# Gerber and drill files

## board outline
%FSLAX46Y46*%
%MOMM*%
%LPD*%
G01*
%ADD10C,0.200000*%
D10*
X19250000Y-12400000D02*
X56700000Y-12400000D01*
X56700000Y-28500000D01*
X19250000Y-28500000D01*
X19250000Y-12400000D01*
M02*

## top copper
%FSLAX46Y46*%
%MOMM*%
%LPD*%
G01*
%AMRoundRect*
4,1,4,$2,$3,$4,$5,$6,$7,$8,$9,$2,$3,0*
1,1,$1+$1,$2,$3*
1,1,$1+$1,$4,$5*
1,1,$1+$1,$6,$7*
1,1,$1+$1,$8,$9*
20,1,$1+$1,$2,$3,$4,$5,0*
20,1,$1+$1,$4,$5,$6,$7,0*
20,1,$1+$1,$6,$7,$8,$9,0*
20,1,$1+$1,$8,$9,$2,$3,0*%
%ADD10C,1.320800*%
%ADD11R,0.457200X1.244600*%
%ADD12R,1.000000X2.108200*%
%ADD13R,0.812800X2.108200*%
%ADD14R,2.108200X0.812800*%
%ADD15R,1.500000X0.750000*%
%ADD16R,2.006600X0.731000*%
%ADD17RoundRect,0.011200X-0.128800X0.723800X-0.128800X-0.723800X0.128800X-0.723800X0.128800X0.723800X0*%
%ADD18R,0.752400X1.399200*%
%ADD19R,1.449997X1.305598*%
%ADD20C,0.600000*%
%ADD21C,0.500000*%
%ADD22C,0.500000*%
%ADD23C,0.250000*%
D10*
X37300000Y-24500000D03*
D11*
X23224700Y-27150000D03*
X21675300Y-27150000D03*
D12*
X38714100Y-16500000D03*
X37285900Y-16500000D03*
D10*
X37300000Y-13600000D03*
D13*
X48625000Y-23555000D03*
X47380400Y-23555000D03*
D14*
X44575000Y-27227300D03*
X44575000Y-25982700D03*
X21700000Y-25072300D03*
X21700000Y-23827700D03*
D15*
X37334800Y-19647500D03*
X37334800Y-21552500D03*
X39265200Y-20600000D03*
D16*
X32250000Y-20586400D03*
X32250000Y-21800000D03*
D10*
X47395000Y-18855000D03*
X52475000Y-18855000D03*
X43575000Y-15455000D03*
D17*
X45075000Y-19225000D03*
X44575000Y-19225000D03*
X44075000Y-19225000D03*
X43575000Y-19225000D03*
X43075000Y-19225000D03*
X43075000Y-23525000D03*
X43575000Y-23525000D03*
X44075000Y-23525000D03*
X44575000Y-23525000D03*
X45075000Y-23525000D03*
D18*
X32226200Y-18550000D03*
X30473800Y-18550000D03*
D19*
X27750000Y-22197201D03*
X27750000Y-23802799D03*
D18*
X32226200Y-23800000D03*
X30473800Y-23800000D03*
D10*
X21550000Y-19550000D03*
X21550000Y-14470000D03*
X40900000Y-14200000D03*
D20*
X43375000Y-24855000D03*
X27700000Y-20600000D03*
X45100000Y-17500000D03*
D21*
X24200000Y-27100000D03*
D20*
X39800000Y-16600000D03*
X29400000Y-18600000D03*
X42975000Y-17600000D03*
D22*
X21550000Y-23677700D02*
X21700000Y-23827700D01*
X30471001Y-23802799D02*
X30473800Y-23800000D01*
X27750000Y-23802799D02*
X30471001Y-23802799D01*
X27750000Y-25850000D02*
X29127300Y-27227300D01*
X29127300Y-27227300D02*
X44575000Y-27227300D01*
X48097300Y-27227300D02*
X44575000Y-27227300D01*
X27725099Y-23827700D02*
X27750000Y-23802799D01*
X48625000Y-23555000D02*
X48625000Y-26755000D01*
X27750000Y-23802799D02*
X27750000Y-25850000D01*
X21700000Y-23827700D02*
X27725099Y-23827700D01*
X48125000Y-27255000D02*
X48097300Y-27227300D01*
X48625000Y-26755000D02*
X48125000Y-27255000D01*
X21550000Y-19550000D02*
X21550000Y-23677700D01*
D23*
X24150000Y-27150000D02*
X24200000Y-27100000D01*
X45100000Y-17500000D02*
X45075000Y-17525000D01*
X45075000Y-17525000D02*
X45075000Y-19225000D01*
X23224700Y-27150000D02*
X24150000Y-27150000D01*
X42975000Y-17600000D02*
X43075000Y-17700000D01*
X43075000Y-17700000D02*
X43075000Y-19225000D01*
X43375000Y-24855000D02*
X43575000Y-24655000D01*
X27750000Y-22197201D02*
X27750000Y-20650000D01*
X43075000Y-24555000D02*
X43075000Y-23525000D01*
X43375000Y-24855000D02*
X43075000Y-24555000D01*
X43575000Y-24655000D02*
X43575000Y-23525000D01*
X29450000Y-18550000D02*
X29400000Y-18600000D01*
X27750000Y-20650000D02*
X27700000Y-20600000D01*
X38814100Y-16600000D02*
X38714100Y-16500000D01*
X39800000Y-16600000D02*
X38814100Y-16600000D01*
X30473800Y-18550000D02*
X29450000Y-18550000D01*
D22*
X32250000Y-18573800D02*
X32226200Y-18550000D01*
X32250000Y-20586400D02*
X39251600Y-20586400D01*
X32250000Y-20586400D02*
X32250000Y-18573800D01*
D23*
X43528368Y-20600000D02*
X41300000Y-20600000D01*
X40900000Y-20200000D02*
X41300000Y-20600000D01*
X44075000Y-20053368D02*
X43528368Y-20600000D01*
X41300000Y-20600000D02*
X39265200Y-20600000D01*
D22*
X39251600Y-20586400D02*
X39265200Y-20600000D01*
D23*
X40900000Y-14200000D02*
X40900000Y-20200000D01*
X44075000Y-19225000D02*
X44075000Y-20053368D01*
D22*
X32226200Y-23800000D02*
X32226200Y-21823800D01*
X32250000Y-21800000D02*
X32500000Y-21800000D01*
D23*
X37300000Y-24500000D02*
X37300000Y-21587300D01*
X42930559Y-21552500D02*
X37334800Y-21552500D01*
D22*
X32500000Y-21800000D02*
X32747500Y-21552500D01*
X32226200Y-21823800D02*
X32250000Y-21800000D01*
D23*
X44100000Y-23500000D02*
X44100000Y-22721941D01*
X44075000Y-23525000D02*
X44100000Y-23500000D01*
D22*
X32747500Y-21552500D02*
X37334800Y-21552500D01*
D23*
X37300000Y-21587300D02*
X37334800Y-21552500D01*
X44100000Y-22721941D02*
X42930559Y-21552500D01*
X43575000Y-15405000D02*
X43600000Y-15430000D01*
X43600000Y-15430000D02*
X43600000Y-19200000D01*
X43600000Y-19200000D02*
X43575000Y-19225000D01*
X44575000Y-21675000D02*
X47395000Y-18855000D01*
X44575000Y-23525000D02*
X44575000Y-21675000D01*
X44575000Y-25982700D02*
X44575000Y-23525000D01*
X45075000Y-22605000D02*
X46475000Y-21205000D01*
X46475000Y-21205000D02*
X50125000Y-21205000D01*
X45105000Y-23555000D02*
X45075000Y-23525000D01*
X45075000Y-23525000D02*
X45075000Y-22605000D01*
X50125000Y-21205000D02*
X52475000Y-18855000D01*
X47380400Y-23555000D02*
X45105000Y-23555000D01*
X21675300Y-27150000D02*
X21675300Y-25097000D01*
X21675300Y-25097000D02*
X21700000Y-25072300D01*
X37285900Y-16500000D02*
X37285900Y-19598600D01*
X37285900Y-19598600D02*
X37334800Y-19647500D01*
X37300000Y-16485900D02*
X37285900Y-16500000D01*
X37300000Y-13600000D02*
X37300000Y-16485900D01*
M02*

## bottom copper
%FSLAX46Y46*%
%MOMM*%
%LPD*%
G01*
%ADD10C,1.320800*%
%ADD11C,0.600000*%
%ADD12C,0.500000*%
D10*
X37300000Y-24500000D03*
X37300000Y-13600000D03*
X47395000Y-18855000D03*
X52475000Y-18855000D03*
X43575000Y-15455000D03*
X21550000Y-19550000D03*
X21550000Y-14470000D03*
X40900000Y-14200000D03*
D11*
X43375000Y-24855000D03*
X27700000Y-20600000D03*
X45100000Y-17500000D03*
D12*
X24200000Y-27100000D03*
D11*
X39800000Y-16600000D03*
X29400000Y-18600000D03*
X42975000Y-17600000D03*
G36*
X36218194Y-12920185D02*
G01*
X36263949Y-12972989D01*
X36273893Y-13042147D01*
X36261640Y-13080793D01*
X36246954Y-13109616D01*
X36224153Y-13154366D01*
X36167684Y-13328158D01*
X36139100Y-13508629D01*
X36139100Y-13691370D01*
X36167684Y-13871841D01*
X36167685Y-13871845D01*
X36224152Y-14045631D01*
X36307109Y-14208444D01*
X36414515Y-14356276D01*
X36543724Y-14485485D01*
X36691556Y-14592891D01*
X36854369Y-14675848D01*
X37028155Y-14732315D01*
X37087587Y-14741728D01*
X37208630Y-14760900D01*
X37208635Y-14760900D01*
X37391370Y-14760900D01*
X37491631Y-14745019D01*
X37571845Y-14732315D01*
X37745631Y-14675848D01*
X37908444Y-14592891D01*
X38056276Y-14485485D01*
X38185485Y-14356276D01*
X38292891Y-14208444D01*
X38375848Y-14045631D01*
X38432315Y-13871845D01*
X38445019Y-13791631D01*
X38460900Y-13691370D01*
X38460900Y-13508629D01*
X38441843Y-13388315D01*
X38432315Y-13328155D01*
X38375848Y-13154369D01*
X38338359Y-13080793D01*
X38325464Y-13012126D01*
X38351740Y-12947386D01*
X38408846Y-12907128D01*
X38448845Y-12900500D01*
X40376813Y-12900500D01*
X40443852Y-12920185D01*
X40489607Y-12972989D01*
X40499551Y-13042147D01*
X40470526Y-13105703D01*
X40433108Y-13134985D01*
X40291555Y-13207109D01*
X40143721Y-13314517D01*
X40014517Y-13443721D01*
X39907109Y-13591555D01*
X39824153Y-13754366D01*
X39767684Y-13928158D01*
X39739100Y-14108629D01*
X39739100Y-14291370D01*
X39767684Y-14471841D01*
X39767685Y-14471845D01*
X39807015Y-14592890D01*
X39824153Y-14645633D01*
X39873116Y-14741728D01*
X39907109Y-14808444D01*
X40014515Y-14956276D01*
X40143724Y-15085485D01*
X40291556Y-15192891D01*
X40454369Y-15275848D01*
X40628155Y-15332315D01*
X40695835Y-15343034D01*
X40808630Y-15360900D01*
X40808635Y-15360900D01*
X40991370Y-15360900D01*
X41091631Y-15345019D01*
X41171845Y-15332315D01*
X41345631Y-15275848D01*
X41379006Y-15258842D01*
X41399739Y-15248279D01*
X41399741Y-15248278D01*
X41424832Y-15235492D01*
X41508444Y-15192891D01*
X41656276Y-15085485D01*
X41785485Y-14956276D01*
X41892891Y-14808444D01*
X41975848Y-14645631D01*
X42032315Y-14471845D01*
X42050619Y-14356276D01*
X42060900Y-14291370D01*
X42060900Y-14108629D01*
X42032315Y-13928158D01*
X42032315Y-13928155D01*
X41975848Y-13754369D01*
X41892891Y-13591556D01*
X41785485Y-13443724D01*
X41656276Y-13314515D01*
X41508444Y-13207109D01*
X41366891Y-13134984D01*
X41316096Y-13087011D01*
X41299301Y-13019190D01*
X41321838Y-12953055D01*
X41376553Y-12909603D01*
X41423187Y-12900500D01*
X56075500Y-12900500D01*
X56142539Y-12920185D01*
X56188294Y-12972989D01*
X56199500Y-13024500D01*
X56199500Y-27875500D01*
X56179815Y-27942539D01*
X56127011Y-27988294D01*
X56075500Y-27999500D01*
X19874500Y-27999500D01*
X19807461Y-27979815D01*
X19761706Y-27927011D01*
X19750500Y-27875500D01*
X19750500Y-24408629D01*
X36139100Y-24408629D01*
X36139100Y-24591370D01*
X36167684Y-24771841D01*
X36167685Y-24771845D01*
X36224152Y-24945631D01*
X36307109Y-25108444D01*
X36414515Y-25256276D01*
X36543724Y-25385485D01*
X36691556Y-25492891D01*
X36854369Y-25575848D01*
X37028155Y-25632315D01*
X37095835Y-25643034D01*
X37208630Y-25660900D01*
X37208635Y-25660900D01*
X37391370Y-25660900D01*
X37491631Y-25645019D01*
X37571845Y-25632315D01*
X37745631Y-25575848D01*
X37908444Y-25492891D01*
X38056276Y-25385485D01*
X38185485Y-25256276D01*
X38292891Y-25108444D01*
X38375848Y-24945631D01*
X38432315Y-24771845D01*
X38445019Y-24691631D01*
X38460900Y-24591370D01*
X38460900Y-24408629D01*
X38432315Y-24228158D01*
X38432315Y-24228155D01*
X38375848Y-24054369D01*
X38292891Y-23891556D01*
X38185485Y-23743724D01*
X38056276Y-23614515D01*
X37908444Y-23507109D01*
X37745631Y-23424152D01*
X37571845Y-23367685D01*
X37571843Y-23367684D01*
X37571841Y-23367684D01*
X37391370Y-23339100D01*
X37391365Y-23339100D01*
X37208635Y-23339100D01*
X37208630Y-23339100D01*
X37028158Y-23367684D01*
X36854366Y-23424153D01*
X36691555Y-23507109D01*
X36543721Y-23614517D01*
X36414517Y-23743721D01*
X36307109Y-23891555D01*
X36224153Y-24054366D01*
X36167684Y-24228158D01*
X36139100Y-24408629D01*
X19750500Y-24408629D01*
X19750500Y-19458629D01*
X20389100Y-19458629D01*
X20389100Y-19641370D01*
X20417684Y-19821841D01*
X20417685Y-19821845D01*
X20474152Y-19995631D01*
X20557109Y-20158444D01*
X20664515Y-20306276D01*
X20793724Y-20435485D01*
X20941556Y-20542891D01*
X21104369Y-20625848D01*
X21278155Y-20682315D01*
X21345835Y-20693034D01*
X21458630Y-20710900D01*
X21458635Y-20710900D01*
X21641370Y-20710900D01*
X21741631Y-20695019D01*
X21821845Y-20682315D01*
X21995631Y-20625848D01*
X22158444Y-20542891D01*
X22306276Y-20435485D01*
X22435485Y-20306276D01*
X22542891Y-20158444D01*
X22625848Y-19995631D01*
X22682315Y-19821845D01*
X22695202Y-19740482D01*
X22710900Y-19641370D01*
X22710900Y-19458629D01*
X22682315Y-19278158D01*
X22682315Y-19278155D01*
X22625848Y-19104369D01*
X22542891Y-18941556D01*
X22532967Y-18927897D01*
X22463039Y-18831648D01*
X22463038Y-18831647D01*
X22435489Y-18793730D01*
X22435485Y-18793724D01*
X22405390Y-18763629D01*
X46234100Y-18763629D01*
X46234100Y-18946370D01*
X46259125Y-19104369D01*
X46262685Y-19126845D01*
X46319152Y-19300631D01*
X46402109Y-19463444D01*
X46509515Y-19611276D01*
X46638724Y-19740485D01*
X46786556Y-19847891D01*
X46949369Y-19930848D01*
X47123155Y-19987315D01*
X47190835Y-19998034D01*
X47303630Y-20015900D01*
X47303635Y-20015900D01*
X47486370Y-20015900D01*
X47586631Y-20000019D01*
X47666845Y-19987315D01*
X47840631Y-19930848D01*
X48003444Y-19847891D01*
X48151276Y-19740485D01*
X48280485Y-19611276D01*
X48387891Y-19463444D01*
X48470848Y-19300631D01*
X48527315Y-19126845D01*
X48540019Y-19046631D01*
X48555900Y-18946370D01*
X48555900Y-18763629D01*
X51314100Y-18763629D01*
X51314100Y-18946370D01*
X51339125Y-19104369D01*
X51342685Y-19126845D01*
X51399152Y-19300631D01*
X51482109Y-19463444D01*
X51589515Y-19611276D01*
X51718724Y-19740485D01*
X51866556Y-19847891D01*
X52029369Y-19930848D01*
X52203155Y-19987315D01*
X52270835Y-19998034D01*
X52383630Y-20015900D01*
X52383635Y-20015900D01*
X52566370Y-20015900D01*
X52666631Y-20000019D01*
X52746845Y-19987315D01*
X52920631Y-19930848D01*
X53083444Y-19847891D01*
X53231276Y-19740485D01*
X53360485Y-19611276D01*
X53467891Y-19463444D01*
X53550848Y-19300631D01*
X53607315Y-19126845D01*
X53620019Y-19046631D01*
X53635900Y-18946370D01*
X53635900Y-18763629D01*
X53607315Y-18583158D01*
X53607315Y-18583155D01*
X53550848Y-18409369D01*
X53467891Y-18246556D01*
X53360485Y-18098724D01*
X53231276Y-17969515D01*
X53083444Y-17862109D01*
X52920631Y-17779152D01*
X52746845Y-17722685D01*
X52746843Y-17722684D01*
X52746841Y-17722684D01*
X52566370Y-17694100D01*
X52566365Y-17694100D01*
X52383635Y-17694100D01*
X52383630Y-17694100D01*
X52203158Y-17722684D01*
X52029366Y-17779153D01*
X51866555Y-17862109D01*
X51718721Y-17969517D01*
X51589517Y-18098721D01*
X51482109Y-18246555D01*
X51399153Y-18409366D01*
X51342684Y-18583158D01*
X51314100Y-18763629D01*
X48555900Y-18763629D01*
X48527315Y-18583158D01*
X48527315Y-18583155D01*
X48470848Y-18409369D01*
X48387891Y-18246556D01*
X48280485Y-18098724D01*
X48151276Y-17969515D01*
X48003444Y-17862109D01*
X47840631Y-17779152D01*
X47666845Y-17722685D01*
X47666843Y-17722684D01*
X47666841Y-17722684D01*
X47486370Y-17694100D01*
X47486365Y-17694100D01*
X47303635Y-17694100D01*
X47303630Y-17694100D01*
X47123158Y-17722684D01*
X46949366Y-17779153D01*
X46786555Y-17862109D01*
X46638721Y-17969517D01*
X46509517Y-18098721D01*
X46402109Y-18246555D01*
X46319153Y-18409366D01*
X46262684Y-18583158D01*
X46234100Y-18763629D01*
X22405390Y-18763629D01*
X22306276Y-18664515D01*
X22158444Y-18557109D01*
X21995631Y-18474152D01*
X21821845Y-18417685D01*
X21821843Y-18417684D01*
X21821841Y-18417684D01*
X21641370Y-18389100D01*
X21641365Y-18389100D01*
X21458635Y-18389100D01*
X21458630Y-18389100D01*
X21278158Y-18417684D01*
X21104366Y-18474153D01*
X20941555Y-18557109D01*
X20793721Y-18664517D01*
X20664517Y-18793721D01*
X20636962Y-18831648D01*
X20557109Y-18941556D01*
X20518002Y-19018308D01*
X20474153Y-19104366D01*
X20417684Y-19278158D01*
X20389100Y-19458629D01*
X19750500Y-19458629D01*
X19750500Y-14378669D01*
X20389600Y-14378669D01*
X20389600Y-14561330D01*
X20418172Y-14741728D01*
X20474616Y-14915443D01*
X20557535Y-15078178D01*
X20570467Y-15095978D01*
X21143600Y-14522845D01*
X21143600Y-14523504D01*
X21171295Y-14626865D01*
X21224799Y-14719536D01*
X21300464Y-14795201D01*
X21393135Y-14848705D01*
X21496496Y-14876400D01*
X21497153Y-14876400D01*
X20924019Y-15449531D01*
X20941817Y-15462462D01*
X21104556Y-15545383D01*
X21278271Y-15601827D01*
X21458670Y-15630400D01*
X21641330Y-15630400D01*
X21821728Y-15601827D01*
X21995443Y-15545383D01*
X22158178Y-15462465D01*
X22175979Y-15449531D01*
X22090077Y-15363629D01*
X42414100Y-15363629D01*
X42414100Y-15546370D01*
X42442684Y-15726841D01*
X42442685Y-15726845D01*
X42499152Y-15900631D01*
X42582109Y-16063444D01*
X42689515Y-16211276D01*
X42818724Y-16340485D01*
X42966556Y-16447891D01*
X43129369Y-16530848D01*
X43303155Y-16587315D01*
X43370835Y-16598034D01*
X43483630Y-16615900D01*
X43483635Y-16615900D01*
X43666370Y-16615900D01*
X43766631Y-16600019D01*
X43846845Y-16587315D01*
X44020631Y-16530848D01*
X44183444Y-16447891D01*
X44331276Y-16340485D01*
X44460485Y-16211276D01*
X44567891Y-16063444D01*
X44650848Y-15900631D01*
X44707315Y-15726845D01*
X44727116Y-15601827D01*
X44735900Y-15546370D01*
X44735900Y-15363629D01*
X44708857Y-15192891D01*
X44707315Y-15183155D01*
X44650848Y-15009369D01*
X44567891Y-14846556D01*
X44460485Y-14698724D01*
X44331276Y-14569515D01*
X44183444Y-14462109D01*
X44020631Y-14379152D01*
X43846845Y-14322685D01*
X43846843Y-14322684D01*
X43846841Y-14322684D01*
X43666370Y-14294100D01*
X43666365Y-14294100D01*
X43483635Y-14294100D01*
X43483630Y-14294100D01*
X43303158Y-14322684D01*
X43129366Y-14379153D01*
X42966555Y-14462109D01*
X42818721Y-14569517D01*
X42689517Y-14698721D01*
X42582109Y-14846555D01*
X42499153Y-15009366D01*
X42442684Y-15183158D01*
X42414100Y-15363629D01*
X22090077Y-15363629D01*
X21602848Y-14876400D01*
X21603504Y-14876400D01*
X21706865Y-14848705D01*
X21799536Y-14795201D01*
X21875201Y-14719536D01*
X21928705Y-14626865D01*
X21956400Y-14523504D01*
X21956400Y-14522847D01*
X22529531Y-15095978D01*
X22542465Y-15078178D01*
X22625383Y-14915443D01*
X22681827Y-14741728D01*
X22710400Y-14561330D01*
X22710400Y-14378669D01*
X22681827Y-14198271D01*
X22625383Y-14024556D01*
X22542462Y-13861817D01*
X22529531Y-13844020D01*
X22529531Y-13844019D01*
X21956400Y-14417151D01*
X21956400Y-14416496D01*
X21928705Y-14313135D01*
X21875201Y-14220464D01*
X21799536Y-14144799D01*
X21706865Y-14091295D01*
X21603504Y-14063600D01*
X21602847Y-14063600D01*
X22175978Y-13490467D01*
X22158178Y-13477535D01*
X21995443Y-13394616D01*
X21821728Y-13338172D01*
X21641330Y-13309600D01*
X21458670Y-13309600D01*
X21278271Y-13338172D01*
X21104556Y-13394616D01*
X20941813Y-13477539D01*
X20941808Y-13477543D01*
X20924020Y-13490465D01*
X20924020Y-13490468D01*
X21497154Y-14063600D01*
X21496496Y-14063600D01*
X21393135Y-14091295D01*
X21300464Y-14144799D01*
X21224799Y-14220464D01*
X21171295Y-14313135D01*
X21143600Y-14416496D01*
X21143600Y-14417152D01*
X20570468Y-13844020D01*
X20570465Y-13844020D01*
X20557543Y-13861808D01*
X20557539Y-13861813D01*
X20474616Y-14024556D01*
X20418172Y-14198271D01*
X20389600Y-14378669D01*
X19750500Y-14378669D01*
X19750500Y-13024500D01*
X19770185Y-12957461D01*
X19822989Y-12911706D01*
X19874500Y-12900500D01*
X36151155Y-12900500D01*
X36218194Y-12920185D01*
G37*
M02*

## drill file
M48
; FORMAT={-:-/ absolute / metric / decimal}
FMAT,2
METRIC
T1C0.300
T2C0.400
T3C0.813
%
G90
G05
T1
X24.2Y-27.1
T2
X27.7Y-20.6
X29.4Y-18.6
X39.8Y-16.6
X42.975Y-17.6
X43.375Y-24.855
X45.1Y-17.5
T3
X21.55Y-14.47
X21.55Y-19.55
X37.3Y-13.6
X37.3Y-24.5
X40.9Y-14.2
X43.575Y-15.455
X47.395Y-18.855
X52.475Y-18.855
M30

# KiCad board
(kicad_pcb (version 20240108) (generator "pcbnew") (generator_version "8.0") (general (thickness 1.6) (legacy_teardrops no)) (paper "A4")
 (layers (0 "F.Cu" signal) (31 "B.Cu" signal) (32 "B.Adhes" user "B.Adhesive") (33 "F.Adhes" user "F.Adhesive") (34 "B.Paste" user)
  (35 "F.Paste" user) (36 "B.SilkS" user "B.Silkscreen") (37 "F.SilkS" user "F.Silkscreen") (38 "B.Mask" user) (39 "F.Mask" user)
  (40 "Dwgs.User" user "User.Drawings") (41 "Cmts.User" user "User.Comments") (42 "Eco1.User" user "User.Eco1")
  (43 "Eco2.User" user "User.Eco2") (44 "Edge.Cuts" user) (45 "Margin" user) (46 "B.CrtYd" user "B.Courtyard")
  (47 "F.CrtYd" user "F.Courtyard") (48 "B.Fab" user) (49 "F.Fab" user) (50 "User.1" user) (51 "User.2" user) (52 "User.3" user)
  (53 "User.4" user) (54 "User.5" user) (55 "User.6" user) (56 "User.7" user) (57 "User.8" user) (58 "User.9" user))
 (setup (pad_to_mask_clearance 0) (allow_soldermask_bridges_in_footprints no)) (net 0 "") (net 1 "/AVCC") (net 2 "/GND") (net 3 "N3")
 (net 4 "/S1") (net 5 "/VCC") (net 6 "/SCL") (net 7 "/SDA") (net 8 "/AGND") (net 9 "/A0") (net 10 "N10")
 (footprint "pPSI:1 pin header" (layer "F.Cu") (at 37.3 24.5)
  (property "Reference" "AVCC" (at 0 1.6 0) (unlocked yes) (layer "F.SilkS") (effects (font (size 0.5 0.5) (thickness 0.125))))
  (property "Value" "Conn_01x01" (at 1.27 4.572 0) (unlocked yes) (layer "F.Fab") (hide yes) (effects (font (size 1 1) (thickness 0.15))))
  (pad "1" thru_hole circle (at 0 0) (size 1.3208 1.3208) (drill 0.8128) (layers "*.Cu" "*.Mask") (remove_unused_layers no) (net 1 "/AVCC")))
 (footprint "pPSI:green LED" (layer "F.Cu") (at 22.45 27.15 180)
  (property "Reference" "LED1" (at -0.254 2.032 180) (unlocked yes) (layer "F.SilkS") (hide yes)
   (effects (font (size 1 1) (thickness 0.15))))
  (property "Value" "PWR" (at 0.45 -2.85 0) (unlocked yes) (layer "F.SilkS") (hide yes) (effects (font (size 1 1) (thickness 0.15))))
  (pad "1" smd rect (at -0.7747 0 180) (size 0.4572 1.2446) (layers "F.Cu" "F.Paste" "F.Mask") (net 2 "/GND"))
  (pad "2" smd rect (at 0.7747 0 180) (size 0.4572 1.2446) (layers "F.Cu" "F.Paste" "F.Mask") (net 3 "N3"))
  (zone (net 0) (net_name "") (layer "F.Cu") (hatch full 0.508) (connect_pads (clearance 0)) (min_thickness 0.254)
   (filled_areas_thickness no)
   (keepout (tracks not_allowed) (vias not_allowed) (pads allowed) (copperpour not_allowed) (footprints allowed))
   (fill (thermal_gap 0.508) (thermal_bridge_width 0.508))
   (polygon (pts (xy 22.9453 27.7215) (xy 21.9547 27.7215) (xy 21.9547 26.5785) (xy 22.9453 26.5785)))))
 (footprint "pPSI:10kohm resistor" (layer "F.Cu") (at 38 16.5 180)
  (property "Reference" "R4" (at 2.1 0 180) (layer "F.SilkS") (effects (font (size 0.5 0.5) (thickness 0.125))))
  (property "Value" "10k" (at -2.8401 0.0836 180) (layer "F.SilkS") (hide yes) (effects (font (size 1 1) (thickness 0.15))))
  (pad "1" smd rect (at -0.7141 0 180) (size 1 2.1082) (layers "F.Cu" "F.Paste" "F.Mask") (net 2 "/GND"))
  (pad "2" smd rect (at 0.7141 0 180) (size 1 2.1082) (layers "F.Cu" "F.Paste" "F.Mask") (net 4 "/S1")))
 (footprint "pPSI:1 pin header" (layer "F.Cu") (at 37.3 13.6 180)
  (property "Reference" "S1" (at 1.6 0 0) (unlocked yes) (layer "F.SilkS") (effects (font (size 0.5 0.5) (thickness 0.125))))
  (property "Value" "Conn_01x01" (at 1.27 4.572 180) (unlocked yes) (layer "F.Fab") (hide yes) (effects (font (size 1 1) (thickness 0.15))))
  (pad "1" thru_hole circle (at 0 0 180) (size 1.3208 1.3208) (drill 0.8128) (layers "*.Cu" "*.Mask") (remove_unused_layers no)
   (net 4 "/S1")))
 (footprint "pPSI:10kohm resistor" (layer "F.Cu") (at 48.0027 23.555 180)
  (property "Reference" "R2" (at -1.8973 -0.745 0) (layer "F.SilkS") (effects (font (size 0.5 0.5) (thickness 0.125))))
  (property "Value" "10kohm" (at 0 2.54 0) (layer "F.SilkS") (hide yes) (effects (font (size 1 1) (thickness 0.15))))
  (pad "1" smd rect (at -0.6223 0 180) (size 0.8128 2.1082) (layers "F.Cu" "F.Paste" "F.Mask") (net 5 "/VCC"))
  (pad "2" smd rect (at 0.6223 0 180) (size 0.8128 2.1082) (layers "F.Cu" "F.Paste" "F.Mask") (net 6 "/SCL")))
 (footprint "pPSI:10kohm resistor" (layer "F.Cu") (at 44.575 26.605 90)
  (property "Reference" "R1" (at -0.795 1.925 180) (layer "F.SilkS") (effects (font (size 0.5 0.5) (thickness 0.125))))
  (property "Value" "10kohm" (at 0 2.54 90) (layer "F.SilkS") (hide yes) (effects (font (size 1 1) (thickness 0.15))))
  (pad "1" smd rect (at -0.6223 0 90) (size 0.8128 2.1082) (layers "F.Cu" "F.Paste" "F.Mask") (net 5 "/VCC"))
  (pad "2" smd rect (at 0.6223 0 90) (size 0.8128 2.1082) (layers "F.Cu" "F.Paste" "F.Mask") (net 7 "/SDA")))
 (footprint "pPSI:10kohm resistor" (layer "F.Cu") (at 21.7 24.45 90)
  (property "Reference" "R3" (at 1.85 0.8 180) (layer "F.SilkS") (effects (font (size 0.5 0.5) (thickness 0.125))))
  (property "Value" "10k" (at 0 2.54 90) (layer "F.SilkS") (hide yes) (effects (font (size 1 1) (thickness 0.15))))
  (pad "1" smd rect (at -0.6223 0 90) (size 0.8128 2.1082) (layers "F.Cu" "F.Paste" "F.Mask") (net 3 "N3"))
  (pad "2" smd rect (at 0.6223 0 90) (size 0.8128 2.1082) (layers "F.Cu" "F.Paste" "F.Mask") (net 5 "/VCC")))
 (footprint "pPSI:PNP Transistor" (layer "F.Cu") (at 38.3 20.6 -90)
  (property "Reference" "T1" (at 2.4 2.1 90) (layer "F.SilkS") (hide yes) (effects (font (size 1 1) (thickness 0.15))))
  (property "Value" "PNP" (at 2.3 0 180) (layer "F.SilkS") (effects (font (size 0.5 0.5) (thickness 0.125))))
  (pad "1" smd rect (at -0.9525 0.9652 270) (size 0.75 1.5) (layers "F.Cu" "F.Paste" "F.Mask") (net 4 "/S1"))
  (pad "2" smd rect (at 0.9525 0.9652 270) (size 0.75 1.5) (layers "F.Cu" "F.Paste" "F.Mask") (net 1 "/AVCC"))
  (pad "3" smd rect (at 0 -0.9652 270) (size 0.75 1.5) (layers "F.Cu" "F.Paste" "F.Mask") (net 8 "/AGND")))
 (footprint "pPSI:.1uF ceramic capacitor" (layer "F.Cu") (at 32.25 21.1932 -90)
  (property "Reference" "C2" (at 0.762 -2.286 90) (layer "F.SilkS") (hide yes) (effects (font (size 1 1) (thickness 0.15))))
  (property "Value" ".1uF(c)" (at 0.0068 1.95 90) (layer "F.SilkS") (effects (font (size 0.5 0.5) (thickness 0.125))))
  (pad "1" smd rect (at -0.6068 0 270) (size 0.731 2.0066) (layers "F.Cu" "F.Paste" "F.Mask") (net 8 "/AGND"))
  (pad "2" smd rect (at 0.6068 0 270) (size 0.731 2.0066) (layers "F.Cu" "F.Paste" "F.Mask") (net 1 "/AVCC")))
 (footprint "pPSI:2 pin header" (layer "F.Cu") (at 47.395 18.855)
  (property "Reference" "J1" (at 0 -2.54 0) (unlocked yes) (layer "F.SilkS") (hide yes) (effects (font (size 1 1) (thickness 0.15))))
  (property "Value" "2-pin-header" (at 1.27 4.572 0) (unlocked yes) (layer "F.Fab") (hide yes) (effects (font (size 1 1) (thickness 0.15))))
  (pad "1" thru_hole circle (at 0 0) (size 1.3208 1.3208) (drill 0.8128) (layers "*.Cu" "*.Mask") (remove_unused_layers no) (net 7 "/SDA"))
  (pad "2" thru_hole circle (at 5.08 0) (size 1.3208 1.3208) (drill 0.8128) (layers "*.Cu" "*.Mask") (remove_unused_layers no)
   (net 6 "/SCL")))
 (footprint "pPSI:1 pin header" (layer "F.Cu") (at 43.575 15.455)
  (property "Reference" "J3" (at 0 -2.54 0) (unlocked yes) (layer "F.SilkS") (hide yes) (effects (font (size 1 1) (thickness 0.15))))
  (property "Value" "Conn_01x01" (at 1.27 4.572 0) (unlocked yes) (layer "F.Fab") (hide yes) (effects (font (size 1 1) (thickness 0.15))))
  (pad "1" thru_hole circle (at 0 0) (size 1.3208 1.3208) (drill 0.8128) (layers "*.Cu" "*.Mask") (remove_unused_layers no) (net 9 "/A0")))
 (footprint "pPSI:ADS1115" (layer "F.Cu") (at 44.075 21.375 -90)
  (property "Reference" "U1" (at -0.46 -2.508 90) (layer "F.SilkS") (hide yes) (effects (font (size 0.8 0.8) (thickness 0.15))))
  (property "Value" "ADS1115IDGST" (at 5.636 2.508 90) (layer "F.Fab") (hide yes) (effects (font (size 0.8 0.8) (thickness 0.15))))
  (pad "1" smd roundrect (at -2.15 -1 270) (size 1.47 0.28) (layers "F.Cu" "F.Paste" "F.Mask") (roundrect_rratio 0.04) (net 2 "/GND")
   (solder_mask_margin 0.102))
  (pad "2" smd roundrect (at -2.15 -0.5 270) (size 1.47 0.28) (layers "F.Cu" "F.Paste" "F.Mask") (roundrect_rratio 0.04) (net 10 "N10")
   (solder_mask_margin 0.102))
  (pad "3" smd roundrect (at -2.15 0 270) (size 1.47 0.28) (layers "F.Cu" "F.Paste" "F.Mask") (roundrect_rratio 0.04) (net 8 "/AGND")
   (solder_mask_margin 0.102))
  (pad "4" smd roundrect (at -2.15 0.5 270) (size 1.47 0.28) (layers "F.Cu" "F.Paste" "F.Mask") (roundrect_rratio 0.04) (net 9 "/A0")
   (solder_mask_margin 0.102))
  (pad "5" smd roundrect (at -2.15 1 270) (size 1.47 0.28) (layers "F.Cu" "F.Paste" "F.Mask") (roundrect_rratio 0.04) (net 2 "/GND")
   (solder_mask_margin 0.102))
  (pad "6" smd roundrect (at 2.15 1 270) (size 1.47 0.28) (layers "F.Cu" "F.Paste" "F.Mask") (roundrect_rratio 0.04) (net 2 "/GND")
   (solder_mask_margin 0.102))
  (pad "7" smd roundrect (at 2.15 0.5 270) (size 1.47 0.28) (layers "F.Cu" "F.Paste" "F.Mask") (roundrect_rratio 0.04) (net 2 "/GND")
   (solder_mask_margin 0.102))
  (pad "8" smd roundrect (at 2.15 0 270) (size 1.47 0.28) (layers "F.Cu" "F.Paste" "F.Mask") (roundrect_rratio 0.04) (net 1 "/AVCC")
   (solder_mask_margin 0.102))
  (pad "9" smd roundrect (at 2.15 -0.5 270) (size 1.47 0.28) (layers "F.Cu" "F.Paste" "F.Mask") (roundrect_rratio 0.04) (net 7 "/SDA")
   (solder_mask_margin 0.102))
  (pad "10" smd roundrect (at 2.15 -1 270) (size 1.47 0.28) (layers "F.Cu" "F.Paste" "F.Mask") (roundrect_rratio 0.04) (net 6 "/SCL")
   (solder_mask_margin 0.102)))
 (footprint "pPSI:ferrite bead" (layer "F.Cu") (at 31.35 18.55 180)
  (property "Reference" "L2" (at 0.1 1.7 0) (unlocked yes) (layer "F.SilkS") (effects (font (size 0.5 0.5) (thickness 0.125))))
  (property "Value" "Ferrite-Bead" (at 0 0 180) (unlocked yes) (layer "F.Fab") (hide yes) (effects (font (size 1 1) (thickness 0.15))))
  (pad "1" smd rect (at -0.8762 0 180) (size 0.7524 1.3992) (layers "F.Cu" "F.Paste" "F.Mask") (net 8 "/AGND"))
  (pad "2" smd rect (at 0.8762 0 180) (size 0.7524 1.3992) (layers "F.Cu" "F.Paste" "F.Mask") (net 2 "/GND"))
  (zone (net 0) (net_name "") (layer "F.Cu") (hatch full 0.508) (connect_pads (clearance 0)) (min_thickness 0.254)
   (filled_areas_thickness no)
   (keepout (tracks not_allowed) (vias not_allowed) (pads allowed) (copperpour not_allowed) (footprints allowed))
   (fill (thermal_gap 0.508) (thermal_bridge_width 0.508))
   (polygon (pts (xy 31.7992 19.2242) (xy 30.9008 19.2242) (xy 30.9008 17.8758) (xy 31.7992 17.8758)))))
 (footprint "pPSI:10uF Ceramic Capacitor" (layer "F.Cu") (at 27.75 23 -90)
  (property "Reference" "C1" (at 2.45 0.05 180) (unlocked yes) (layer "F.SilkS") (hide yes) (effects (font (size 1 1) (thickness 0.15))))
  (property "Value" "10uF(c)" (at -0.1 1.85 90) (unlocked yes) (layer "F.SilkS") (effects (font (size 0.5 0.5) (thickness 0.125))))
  (pad "1" smd rect (at -0.802799 0 270) (size 1.305598 1.449997) (layers "F.Cu" "F.Paste" "F.Mask") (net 2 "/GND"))
  (pad "2" smd rect (at 0.802799 0 270) (size 1.305598 1.449997) (layers "F.Cu" "F.Paste" "F.Mask") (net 5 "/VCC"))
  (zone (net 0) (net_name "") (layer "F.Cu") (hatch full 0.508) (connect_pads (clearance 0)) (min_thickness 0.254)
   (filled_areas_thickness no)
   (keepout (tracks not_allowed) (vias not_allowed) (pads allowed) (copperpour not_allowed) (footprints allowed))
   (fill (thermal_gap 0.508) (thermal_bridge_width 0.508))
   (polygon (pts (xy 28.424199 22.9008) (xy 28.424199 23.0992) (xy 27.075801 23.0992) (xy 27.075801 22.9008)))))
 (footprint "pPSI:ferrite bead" (layer "F.Cu") (at 31.35 23.8 180)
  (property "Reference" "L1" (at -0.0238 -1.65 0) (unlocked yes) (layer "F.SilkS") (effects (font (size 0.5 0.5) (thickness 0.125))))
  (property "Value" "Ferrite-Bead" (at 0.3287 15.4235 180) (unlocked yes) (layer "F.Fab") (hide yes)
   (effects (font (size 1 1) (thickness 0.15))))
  (pad "1" smd rect (at -0.8762 0 180) (size 0.7524 1.3992) (layers "F.Cu" "F.Paste" "F.Mask") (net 1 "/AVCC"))
  (pad "2" smd rect (at 0.8762 0 180) (size 0.7524 1.3992) (layers "F.Cu" "F.Paste" "F.Mask") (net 5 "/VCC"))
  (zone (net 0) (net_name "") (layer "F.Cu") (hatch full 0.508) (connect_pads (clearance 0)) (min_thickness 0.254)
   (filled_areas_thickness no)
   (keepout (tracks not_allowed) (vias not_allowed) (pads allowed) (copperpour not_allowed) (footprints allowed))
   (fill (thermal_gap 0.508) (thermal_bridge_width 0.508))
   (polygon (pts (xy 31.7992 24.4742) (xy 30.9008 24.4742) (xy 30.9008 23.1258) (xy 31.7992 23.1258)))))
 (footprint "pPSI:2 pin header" (layer "F.Cu") (at 21.55 19.55 90)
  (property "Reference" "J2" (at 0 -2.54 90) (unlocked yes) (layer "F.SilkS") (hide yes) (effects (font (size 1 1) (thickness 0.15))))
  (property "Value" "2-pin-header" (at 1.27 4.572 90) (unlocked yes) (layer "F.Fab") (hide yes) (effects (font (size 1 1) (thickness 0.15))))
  (pad "1" thru_hole circle (at 0 0 90) (size 1.3208 1.3208) (drill 0.8128) (layers "*.Cu" "*.Mask") (remove_unused_layers no)
   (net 5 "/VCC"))
  (pad "2" thru_hole circle (at 5.08 0 90) (size 1.3208 1.3208) (drill 0.8128) (layers "*.Cu" "*.Mask") (remove_unused_layers no)
   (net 2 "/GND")))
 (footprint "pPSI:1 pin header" (layer "F.Cu") (at 40.9 14.2 180)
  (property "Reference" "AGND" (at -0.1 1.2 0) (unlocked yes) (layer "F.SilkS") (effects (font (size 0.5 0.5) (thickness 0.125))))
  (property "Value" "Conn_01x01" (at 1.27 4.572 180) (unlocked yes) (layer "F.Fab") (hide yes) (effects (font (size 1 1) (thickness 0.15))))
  (pad "1" thru_hole circle (at 0 0 180) (size 1.3208 1.3208) (drill 0.8128) (layers "*.Cu" "*.Mask") (remove_unused_layers no)
   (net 8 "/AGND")))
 (gr_rect (start 19.25 12.4) (end 56.7 28.5) (stroke (width 0.2) (type solid)) (fill none) (layer "Edge.Cuts"))
 (segment (start 21.55 23.6777) (end 21.7 23.8277) (width 0.5) (layer "F.Cu") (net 5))
 (segment (start 30.471001 23.802799) (end 30.4738 23.8) (width 0.5) (layer "F.Cu") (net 5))
 (segment (start 27.75 23.802799) (end 30.471001 23.802799) (width 0.5) (layer "F.Cu") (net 5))
 (segment (start 27.75 25.85) (end 29.1273 27.2273) (width 0.5) (layer "F.Cu") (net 5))
 (segment (start 29.1273 27.2273) (end 44.575 27.2273) (width 0.5) (layer "F.Cu") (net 5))
 (segment (start 48.0973 27.2273) (end 44.575 27.2273) (width 0.5) (layer "F.Cu") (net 5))
 (segment (start 27.725099 23.8277) (end 27.75 23.802799) (width 0.5) (layer "F.Cu") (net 5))
 (segment (start 48.625 23.555) (end 48.625 26.755) (width 0.5) (layer "F.Cu") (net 5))
 (segment (start 27.75 23.802799) (end 27.75 25.85) (width 0.5) (layer "F.Cu") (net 5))
 (segment (start 21.7 23.8277) (end 27.725099 23.8277) (width 0.5) (layer "F.Cu") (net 5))
 (segment (start 48.125 27.255) (end 48.0973 27.2273) (width 0.5) (layer "F.Cu") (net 5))
 (segment (start 48.625 26.755) (end 48.125 27.255) (width 0.5) (layer "F.Cu") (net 5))
 (segment (start 21.55 19.55) (end 21.55 23.6777) (width 0.5) (layer "F.Cu") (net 5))
 (segment (start 24.15 27.15) (end 24.2 27.1) (width 0.25) (layer "F.Cu") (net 2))
 (segment (start 45.1 17.5) (end 45.075 17.525) (width 0.25) (layer "F.Cu") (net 2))
 (segment (start 45.075 17.525) (end 45.075 19.225) (width 0.25) (layer "F.Cu") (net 2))
 (segment (start 23.2247 27.15) (end 24.15 27.15) (width 0.25) (layer "F.Cu") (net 2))
 (segment (start 42.975 17.6) (end 43.075 17.7) (width 0.25) (layer "F.Cu") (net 2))
 (segment (start 43.075 17.7) (end 43.075 19.225) (width 0.25) (layer "F.Cu") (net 2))
 (segment (start 43.375 24.855) (end 43.575 24.655) (width 0.25) (layer "F.Cu") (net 2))
 (segment (start 27.75 22.197201) (end 27.75 20.65) (width 0.25) (layer "F.Cu") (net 2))
 (segment (start 43.075 24.555) (end 43.075 23.525) (width 0.25) (layer "F.Cu") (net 2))
 (segment (start 43.375 24.855) (end 43.075 24.555) (width 0.25) (layer "F.Cu") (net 2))
 (segment (start 43.575 24.655) (end 43.575 23.525) (width 0.25) (layer "F.Cu") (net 2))
 (segment (start 29.45 18.55) (end 29.4 18.6) (width 0.25) (layer "F.Cu") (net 2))
 (segment (start 27.75 20.65) (end 27.7 20.6) (width 0.25) (layer "F.Cu") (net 2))
 (segment (start 38.8141 16.6) (end 38.7141 16.5) (width 0.25) (layer "F.Cu") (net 2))
 (segment (start 39.8 16.6) (end 38.8141 16.6) (width 0.25) (layer "F.Cu") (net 2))
 (segment (start 30.4738 18.55) (end 29.45 18.55) (width 0.25) (layer "F.Cu") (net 2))
 (via blind (at 43.375 24.855) (size 0.6) (drill 0.4) (layers "F.Cu" "B.Cu") (free yes) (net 2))
 (via blind (at 27.7 20.6) (size 0.6) (drill 0.4) (layers "F.Cu" "B.Cu") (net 2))
 (via blind (at 45.1 17.5) (size 0.6) (drill 0.4) (layers "F.Cu" "B.Cu") (free yes) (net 2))
 (via blind (at 24.2 27.1) (size 0.5) (drill 0.3) (layers "F.Cu" "B.Cu") (free yes) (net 2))
 (via blind (at 39.8 16.6) (size 0.6) (drill 0.4) (layers "F.Cu" "B.Cu") (free yes) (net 2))
 (via blind (at 29.4 18.6) (size 0.6) (drill 0.4) (layers "F.Cu" "B.Cu") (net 2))
 (via blind (at 42.975 17.6) (size 0.6) (drill 0.4) (layers "F.Cu" "B.Cu") (free yes) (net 2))
 (segment (start 32.25 18.5738) (end 32.2262 18.55) (width 0.5) (layer "F.Cu") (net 8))
 (segment (start 32.25 20.5864) (end 39.2516 20.5864) (width 0.5) (layer "F.Cu") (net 8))
 (segment (start 32.25 20.5864) (end 32.25 18.5738) (width 0.5) (layer "F.Cu") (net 8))
 (segment (start 43.528368 20.6) (end 41.3 20.6) (width 0.25) (layer "F.Cu") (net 8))
 (segment (start 40.9 20.2) (end 41.3 20.6) (width 0.25) (layer "F.Cu") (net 8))
 (segment (start 44.075 20.053368) (end 43.528368 20.6) (width 0.25) (layer "F.Cu") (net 8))
 (segment (start 41.3 20.6) (end 39.2652 20.6) (width 0.25) (layer "F.Cu") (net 8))
 (segment (start 39.2516 20.5864) (end 39.2652 20.6) (width 0.5) (layer "F.Cu") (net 8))
 (segment (start 40.9 14.2) (end 40.9 20.2) (width 0.25) (layer "F.Cu") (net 8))
 (segment (start 44.075 19.225) (end 44.075 20.053368) (width 0.25) (layer "F.Cu") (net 8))
 (segment (start 32.2262 23.8) (end 32.2262 21.8238) (width 0.5) (layer "F.Cu") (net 1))
 (segment (start 32.25 21.8) (end 32.5 21.8) (width 0.5) (layer "F.Cu") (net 1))
 (segment (start 37.3 24.5) (end 37.3 21.5873) (width 0.25) (layer "F.Cu") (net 1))
 (segment (start 42.930559 21.5525) (end 37.3348 21.5525) (width 0.25) (layer "F.Cu") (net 1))
 (segment (start 32.5 21.8) (end 32.7475 21.5525) (width 0.5) (layer "F.Cu") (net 1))
 (segment (start 32.2262 21.8238) (end 32.25 21.8) (width 0.5) (layer "F.Cu") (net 1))
 (segment (start 44.1 23.5) (end 44.1 22.721941) (width 0.25) (layer "F.Cu") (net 1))
 (segment (start 44.075 23.525) (end 44.1 23.5) (width 0.25) (layer "F.Cu") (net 1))
 (segment (start 32.7475 21.5525) (end 37.3348 21.5525) (width 0.5) (layer "F.Cu") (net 1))
 (segment (start 37.3 21.5873) (end 37.3348 21.5525) (width 0.25) (layer "F.Cu") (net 1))
 (segment (start 44.1 22.721941) (end 42.930559 21.5525) (width 0.25) (layer "F.Cu") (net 1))
 (segment (start 43.575 15.405) (end 43.6 15.43) (width 0.25) (layer "F.Cu") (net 9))
 (segment (start 43.6 15.43) (end 43.6 19.2) (width 0.25) (layer "F.Cu") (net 9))
 (segment (start 43.6 19.2) (end 43.575 19.225) (width 0.25) (layer "F.Cu") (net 9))
 (segment (start 44.575 21.675) (end 47.395 18.855) (width 0.25) (layer "F.Cu") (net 7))
 (segment (start 44.575 23.525) (end 44.575 21.675) (width 0.25) (layer "F.Cu") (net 7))
 (segment (start 44.575 25.9827) (end 44.575 23.525) (width 0.25) (layer "F.Cu") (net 7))
 (segment (start 45.075 22.605) (end 46.475 21.205) (width 0.25) (layer "F.Cu") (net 6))
 (segment (start 46.475 21.205) (end 50.125 21.205) (width 0.25) (layer "F.Cu") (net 6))
 (segment (start 45.105 23.555) (end 45.075 23.525) (width 0.25) (layer "F.Cu") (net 6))
 (segment (start 45.075 23.525) (end 45.075 22.605) (width 0.25) (layer "F.Cu") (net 6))
 (segment (start 50.125 21.205) (end 52.475 18.855) (width 0.25) (layer "F.Cu") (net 6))
 (segment (start 47.3804 23.555) (end 45.105 23.555) (width 0.25) (layer "F.Cu") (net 6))
 (segment (start 21.6753 27.15) (end 21.6753 25.097) (width 0.25) (layer "F.Cu") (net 3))
 (segment (start 21.6753 25.097) (end 21.7 25.0723) (width 0.25) (layer "F.Cu") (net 3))
 (segment (start 37.2859 16.5) (end 37.2859 19.5986) (width 0.25) (layer "F.Cu") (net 4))
 (segment (start 37.2859 19.5986) (end 37.3348 19.6475) (width 0.25) (layer "F.Cu") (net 4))
 (segment (start 37.3 16.4859) (end 37.2859 16.5) (width 0.25) (layer "F.Cu") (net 4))
 (segment (start 37.3 13.6) (end 37.3 16.4859) (width 0.25) (layer "F.Cu") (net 4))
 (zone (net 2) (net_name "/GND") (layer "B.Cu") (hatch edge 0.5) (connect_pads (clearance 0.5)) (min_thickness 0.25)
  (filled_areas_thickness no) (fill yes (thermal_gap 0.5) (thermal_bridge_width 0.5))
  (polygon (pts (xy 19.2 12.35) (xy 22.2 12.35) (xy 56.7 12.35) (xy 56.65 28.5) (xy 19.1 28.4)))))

